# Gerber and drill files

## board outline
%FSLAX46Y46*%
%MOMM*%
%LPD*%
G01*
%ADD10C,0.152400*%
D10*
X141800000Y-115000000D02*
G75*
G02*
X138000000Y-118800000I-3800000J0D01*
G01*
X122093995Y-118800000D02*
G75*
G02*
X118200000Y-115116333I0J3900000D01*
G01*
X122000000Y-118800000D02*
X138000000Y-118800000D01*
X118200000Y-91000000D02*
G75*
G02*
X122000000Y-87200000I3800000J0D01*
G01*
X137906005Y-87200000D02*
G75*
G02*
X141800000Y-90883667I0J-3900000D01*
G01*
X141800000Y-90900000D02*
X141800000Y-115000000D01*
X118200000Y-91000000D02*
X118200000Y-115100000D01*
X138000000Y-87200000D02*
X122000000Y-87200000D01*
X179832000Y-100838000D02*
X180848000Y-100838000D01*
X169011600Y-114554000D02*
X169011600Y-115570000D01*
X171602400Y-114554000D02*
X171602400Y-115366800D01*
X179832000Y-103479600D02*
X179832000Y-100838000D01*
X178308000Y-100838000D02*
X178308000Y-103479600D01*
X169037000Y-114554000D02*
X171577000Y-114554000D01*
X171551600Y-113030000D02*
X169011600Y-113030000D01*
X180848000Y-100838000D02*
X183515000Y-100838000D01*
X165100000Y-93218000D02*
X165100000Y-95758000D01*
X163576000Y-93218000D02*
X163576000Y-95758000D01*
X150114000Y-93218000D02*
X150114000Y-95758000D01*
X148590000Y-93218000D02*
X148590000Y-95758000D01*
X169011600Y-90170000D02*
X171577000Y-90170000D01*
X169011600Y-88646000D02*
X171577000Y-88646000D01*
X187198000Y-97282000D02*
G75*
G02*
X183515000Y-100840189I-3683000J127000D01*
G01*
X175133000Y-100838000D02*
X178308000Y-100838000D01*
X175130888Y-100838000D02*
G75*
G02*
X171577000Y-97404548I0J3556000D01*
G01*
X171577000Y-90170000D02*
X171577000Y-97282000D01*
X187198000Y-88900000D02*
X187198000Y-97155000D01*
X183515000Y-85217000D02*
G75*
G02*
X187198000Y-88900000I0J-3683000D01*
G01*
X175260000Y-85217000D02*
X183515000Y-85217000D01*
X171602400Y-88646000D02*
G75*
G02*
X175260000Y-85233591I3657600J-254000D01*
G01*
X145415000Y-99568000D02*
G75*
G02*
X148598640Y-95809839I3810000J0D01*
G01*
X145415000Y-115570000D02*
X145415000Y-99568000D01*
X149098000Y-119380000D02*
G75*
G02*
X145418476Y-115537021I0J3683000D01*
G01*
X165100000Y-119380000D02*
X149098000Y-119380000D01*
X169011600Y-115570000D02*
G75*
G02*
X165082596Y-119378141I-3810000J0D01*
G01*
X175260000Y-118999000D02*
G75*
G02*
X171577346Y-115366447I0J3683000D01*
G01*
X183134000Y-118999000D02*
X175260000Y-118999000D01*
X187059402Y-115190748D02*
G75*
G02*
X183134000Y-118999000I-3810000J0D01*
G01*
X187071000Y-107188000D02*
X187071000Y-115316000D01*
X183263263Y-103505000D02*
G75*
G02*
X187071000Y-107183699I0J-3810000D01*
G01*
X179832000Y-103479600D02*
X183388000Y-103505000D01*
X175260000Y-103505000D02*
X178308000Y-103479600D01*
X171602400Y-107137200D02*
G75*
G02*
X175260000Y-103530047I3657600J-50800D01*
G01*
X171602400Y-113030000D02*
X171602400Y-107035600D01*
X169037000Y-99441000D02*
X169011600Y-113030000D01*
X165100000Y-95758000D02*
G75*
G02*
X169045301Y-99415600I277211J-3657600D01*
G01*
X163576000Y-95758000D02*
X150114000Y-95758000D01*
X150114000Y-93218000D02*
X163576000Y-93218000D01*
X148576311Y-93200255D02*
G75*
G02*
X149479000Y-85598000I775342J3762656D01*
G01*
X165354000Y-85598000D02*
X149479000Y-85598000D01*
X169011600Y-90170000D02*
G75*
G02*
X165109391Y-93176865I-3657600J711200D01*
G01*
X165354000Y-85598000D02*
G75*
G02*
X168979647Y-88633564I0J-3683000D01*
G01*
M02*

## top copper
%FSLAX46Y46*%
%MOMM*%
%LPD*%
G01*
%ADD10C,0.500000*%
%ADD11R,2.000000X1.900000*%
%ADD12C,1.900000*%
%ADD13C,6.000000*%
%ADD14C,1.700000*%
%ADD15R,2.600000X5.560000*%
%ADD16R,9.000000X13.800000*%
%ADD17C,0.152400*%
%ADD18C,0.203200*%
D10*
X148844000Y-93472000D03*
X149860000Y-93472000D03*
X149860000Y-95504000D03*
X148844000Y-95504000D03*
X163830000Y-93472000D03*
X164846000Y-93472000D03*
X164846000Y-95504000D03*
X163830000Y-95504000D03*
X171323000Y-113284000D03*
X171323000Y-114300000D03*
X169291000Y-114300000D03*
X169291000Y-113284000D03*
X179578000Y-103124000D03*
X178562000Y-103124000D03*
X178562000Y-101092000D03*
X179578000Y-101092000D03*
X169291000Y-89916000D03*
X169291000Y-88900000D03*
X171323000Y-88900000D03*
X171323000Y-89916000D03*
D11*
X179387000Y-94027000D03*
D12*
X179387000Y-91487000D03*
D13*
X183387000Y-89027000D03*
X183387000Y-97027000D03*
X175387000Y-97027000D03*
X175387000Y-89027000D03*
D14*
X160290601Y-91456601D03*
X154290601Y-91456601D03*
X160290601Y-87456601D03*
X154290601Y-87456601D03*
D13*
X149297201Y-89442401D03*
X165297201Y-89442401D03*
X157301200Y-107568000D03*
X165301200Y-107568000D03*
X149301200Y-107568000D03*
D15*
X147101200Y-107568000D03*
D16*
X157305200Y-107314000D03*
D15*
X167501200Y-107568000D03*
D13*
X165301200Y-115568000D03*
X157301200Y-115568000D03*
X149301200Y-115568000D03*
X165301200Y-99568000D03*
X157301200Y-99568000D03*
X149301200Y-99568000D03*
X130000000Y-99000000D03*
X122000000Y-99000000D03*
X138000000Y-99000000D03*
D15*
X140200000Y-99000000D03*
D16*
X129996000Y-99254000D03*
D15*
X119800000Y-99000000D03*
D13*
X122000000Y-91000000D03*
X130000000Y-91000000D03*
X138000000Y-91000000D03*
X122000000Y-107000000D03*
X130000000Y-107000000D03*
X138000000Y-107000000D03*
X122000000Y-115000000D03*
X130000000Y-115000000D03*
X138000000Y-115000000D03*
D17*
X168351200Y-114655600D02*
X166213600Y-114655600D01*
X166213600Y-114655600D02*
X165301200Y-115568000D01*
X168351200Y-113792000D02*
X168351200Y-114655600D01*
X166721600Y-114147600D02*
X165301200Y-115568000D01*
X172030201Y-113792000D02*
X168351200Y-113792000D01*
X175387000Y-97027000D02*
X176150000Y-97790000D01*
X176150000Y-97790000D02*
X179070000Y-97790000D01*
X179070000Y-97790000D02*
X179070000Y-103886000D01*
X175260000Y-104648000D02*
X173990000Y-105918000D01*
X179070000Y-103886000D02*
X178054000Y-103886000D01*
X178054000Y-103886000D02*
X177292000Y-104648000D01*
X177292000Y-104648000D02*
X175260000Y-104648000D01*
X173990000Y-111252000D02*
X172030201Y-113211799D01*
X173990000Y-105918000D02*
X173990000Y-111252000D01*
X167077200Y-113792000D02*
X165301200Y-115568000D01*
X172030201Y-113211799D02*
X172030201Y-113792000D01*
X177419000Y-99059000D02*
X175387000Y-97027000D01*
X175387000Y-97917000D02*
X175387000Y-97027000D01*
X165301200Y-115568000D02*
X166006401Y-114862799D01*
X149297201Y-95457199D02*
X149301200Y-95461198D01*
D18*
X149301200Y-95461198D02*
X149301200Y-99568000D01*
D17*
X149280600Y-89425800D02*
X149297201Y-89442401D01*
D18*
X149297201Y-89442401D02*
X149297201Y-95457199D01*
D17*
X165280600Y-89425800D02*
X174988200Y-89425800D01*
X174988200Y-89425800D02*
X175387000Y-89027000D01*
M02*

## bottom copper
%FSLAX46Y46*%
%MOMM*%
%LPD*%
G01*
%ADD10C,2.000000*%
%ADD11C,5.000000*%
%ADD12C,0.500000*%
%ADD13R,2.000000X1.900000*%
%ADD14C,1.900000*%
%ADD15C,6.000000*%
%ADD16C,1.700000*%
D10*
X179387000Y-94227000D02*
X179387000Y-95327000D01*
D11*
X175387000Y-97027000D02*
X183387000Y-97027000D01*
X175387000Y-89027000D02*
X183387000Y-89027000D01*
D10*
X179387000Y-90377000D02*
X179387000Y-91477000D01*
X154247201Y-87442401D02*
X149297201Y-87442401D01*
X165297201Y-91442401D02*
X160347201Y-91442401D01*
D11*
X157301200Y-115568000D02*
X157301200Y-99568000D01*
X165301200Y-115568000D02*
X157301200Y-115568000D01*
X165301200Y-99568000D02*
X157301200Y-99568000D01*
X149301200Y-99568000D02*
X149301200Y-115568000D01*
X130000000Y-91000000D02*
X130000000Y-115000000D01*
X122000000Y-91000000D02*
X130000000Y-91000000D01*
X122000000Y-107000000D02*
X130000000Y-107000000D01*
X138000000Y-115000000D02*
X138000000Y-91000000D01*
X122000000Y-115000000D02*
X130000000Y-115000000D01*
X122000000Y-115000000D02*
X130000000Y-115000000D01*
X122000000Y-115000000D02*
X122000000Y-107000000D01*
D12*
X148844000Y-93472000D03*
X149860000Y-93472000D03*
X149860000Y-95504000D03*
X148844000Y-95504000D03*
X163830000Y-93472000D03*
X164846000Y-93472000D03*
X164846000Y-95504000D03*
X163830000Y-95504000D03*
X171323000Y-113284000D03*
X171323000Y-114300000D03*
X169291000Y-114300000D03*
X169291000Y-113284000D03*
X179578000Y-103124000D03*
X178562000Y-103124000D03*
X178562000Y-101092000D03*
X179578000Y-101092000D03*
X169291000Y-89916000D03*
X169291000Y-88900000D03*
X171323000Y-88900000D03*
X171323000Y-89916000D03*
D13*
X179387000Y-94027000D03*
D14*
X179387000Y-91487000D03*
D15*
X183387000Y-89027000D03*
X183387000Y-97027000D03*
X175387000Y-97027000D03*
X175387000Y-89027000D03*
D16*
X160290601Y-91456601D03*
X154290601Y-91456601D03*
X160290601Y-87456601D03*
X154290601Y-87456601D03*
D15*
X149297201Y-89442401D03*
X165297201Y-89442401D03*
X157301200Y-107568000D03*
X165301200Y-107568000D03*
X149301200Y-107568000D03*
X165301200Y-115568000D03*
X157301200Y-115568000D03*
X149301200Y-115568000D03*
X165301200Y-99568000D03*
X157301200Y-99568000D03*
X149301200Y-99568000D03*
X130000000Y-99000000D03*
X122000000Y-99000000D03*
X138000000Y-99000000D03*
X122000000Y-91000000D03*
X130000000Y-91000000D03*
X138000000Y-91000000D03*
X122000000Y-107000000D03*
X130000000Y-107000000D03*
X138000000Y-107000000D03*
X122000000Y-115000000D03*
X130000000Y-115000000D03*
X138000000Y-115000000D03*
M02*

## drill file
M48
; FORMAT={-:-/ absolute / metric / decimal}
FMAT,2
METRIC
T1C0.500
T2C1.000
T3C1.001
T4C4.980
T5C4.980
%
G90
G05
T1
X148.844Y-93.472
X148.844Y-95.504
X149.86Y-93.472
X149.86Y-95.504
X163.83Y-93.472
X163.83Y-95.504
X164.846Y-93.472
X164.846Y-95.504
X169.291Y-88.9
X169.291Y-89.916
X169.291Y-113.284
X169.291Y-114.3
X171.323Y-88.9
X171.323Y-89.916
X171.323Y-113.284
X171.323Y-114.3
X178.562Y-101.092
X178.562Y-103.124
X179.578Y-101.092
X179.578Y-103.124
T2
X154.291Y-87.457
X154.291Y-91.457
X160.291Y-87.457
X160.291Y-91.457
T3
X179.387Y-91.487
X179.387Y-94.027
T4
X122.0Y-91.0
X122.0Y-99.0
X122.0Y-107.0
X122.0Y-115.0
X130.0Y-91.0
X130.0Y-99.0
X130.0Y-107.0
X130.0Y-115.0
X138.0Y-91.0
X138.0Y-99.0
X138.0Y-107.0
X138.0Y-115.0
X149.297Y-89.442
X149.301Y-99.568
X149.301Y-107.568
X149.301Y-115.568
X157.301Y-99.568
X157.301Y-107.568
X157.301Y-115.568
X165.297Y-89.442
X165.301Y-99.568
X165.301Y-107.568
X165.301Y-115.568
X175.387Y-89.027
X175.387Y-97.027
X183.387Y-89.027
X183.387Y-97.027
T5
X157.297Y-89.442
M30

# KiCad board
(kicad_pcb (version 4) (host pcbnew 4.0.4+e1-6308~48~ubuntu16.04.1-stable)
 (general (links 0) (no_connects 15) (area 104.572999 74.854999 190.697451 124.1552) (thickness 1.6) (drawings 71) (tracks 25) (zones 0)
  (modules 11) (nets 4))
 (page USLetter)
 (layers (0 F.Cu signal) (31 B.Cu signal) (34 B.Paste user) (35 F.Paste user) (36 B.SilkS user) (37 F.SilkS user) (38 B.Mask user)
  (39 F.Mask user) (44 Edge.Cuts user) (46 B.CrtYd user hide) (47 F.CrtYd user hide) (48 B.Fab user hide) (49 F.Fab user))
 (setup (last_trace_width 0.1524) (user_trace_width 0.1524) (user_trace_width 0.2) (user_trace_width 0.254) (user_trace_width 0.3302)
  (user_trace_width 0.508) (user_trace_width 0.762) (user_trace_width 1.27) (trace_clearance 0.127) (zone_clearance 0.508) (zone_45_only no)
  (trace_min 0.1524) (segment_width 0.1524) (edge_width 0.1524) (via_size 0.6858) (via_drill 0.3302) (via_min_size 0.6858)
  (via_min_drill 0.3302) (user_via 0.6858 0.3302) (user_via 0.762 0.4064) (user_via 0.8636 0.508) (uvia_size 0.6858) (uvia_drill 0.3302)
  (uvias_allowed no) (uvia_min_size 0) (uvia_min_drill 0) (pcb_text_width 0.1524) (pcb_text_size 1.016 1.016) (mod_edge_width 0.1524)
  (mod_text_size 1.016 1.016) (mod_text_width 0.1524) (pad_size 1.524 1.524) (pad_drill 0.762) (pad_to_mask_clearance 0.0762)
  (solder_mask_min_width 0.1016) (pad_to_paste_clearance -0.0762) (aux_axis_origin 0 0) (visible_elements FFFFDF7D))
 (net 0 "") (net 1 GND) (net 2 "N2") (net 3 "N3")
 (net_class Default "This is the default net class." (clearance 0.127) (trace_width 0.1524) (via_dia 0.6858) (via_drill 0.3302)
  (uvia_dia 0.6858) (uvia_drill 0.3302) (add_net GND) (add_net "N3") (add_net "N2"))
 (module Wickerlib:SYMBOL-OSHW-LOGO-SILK (layer F.Cu) (at 179.832 109.982)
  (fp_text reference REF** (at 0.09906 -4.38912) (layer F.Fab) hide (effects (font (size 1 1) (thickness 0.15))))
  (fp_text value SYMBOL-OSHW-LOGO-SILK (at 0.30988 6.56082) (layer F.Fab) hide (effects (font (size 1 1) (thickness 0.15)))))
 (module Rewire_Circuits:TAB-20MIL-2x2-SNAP (layer F.Cu) (at 149.352 94.488)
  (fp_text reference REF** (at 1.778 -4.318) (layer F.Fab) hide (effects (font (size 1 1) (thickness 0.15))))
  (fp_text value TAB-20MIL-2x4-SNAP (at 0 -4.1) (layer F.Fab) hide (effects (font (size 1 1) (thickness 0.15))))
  (pad 1 thru_hole circle (at -0.508 -1.016) (size 0.5 0.5) (drill 0.5) (layers *.Cu))
  (pad 1 thru_hole circle (at 0.508 -1.016) (size 0.5 0.5) (drill 0.5) (layers *.Cu))
  (pad 1 thru_hole circle (at 0.508 1.016) (size 0.5 0.5) (drill 0.5) (layers *.Cu))
  (pad 1 thru_hole circle (at -0.508 1.016) (size 0.5 0.5) (drill 0.5) (layers *.Cu)))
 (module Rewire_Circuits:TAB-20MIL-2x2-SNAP (layer F.Cu) (at 164.338 94.488)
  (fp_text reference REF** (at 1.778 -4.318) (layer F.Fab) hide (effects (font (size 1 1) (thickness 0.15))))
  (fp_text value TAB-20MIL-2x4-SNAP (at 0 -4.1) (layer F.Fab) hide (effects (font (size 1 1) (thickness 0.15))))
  (pad 1 thru_hole circle (at -0.508 -1.016) (size 0.5 0.5) (drill 0.5) (layers *.Cu))
  (pad 1 thru_hole circle (at 0.508 -1.016) (size 0.5 0.5) (drill 0.5) (layers *.Cu))
  (pad 1 thru_hole circle (at 0.508 1.016) (size 0.5 0.5) (drill 0.5) (layers *.Cu))
  (pad 1 thru_hole circle (at -0.508 1.016) (size 0.5 0.5) (drill 0.5) (layers *.Cu)))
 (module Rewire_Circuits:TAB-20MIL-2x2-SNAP (layer F.Cu) (at 170.307 113.792 270)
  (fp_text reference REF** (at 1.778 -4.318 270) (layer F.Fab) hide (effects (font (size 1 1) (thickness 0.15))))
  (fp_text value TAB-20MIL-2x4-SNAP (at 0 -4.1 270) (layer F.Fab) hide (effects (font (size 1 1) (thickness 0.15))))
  (pad 1 thru_hole circle (at -0.508 -1.016 270) (size 0.5 0.5) (drill 0.5) (layers *.Cu))
  (pad 1 thru_hole circle (at 0.508 -1.016 270) (size 0.5 0.5) (drill 0.5) (layers *.Cu))
  (pad 1 thru_hole circle (at 0.508 1.016 270) (size 0.5 0.5) (drill 0.5) (layers *.Cu))
  (pad 1 thru_hole circle (at -0.508 1.016 270) (size 0.5 0.5) (drill 0.5) (layers *.Cu)))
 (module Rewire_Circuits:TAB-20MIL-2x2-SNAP (layer F.Cu) (at 179.07 102.108 180)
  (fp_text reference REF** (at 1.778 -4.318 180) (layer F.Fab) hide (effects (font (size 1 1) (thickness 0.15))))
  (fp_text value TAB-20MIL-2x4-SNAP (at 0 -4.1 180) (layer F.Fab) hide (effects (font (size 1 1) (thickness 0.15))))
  (pad 1 thru_hole circle (at -0.508 -1.016 180) (size 0.5 0.5) (drill 0.5) (layers *.Cu))
  (pad 1 thru_hole circle (at 0.508 -1.016 180) (size 0.5 0.5) (drill 0.5) (layers *.Cu))
  (pad 1 thru_hole circle (at 0.508 1.016 180) (size 0.5 0.5) (drill 0.5) (layers *.Cu))
  (pad 1 thru_hole circle (at -0.508 1.016 180) (size 0.5 0.5) (drill 0.5) (layers *.Cu)))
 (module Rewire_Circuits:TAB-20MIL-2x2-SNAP (layer F.Cu) (at 170.307 89.408 90)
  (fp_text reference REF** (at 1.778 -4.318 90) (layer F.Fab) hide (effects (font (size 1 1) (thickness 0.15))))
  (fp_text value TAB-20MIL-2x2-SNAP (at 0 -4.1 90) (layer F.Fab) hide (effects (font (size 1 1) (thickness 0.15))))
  (pad 1 thru_hole circle (at -0.508 -1.016 90) (size 0.5 0.5) (drill 0.5) (layers *.Cu))
  (pad 1 thru_hole circle (at 0.508 -1.016 90) (size 0.5 0.5) (drill 0.5) (layers *.Cu))
  (pad 1 thru_hole circle (at 0.508 1.016 90) (size 0.5 0.5) (drill 0.5) (layers *.Cu))
  (pad 1 thru_hole circle (at -0.508 1.016 90) (size 0.5 0.5) (drill 0.5) (layers *.Cu)))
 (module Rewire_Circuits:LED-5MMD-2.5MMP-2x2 (layer F.Cu) (at 183.387 89.027 180)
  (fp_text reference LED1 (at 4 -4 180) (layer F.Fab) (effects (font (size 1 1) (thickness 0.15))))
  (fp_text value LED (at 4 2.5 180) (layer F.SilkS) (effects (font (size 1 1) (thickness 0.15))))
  (fp_line (start 4 -5.2) (end 4 -6.3) (layer B.Cu) (width 2)) (fp_line (start 8 -8) (end 0 -8) (layer B.Cu) (width 5))
  (fp_line (start 8 0) (end 0 0) (layer B.Cu) (width 5))
  (fp_line (start 4 -1.35) (end 4 -2.45) (layer B.Cu) (width 2))
  (pad - thru_hole rect (at 4 -5 180) (size 2 1.9) (drill 1.00076) (layers *.Cu *.Mask) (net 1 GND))
  (pad + thru_hole circle (at 4 -2.46 90) (size 1.9 1.9) (drill 1.00076) (layers *.Cu *.Mask) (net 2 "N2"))
  (pad + thru_hole circle (at 0 0 180) (size 6 6) (drill 4.98) (layers *.Cu *.Mask) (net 2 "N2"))
  (pad - thru_hole circle (at 0 -8 180) (size 6 6) (drill 4.98) (layers *.Cu *.Mask) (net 1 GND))
  (pad - thru_hole circle (at 8 -8 180) (size 6 6) (drill 4.98) (layers *.Cu *.Mask) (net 1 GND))
  (pad + thru_hole circle (at 8 0 180) (size 6 6) (drill 4.98) (layers *.Cu *.Mask) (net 2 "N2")))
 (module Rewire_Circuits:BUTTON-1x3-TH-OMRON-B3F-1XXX (layer F.Cu) (at 149.297201 89.442401)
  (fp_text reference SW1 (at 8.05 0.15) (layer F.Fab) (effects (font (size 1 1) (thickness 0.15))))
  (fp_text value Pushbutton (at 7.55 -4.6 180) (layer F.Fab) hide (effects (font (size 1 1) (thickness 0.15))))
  (fp_line (start 4.95 -2) (end 0 -2) (layer B.Cu) (width 2)) (fp_line (start 16 2) (end 11.05 2) (layer B.Cu) (width 2))
  (pad 2 thru_hole circle (at 10.9934 2.0142) (size 1.7 1.7) (drill 1) (layers *.Cu *.Mask) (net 2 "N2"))
  (pad 2 thru_hole circle (at 4.9934 2.0142) (size 1.7 1.7) (drill 1) (layers *.Cu *.Mask) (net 2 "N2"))
  (pad 1 thru_hole circle (at 10.9934 -1.9858) (size 1.7 1.7) (drill 1) (layers *.Cu *.Mask) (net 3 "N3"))
  (pad 1 thru_hole circle (at 4.9934 -1.9858) (size 1.7 1.7) (drill 1) (layers *.Cu *.Mask) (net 3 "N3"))
  (pad "" np_thru_hole circle (at 8 0) (size 4.88 4.88) (drill 4.98) (layers *.Cu *.Mask F.SilkS))
  (pad 1 thru_hole circle (at 0 0) (size 6 6) (drill 4.98) (layers *.Cu *.Mask F.SilkS) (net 3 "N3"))
  (pad 2 thru_hole circle (at 16 0) (size 6 6) (drill 4.98) (layers *.Cu *.Mask F.SilkS) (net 2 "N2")))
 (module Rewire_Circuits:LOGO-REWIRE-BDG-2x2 (layer F.Cu) (at 179.324 111.252)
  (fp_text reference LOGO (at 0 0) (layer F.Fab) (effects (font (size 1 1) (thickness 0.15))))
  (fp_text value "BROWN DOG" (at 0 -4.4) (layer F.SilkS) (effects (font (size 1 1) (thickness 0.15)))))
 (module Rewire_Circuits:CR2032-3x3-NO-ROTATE (layer F.Cu) (at 165.3012 99.568 180)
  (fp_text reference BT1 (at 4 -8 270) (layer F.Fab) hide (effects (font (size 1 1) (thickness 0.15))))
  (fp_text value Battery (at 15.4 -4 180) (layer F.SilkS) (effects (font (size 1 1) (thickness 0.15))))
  (fp_line (start 8 -16) (end 8 0) (layer B.Cu) (width 5)) (fp_line (start 0 -16) (end 8 -16) (layer B.Cu) (width 5))
  (fp_line (start 0 0) (end 8 0) (layer B.Cu) (width 5)) (fp_line (start 16 0) (end 16 -16) (layer B.Cu) (width 5))
  (pad GND thru_hole circle (at 8 -8 180) (size 6 6) (drill 4.98) (layers *.Cu *.Mask) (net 1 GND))
  (pad + thru_hole circle (at 0 -8 180) (size 6 6) (drill 4.98) (layers *.Cu) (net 3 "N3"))
  (pad + thru_hole circle (at 16 -8 180) (size 6 6) (drill 4.98) (layers *.Cu B.Mask) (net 3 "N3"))
  (pad + smd rect (at 18.2 -8 180) (size 2.6 5.56) (layers F.Cu F.Paste F.Mask) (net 3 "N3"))
  (pad GND smd rect (at 7.996 -7.746 180) (size 9 13.8) (layers F.Cu F.Paste F.Mask) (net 1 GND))
  (pad + smd rect (at -2.2 -8 180) (size 2.6 5.56) (layers F.Cu F.Paste F.Mask) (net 3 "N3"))
  (pad GND thru_hole circle (at 0 -16 180) (size 6 6) (drill 4.98) (layers *.Cu *.Mask) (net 1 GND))
  (pad GND thru_hole circle (at 8 -16 180) (size 6 6) (drill 4.98) (layers *.Cu *.Mask) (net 1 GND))
  (pad + thru_hole circle (at 16 -16 180) (size 6 6) (drill 4.98) (layers *.Cu B.Mask) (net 3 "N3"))
  (pad GND thru_hole circle (at 0 0 180) (size 6 6) (drill 4.98) (layers *.Cu *.Mask) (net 1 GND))
  (pad GND thru_hole circle (at 8 0 180) (size 6 6) (drill 4.98) (layers *.Cu *.Mask) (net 1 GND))
  (pad + thru_hole circle (at 16 0 180) (size 6 6) (drill 4.98) (layers *.Cu B.Mask) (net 3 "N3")))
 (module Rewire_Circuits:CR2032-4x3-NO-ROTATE (layer F.Cu) (at 122 107)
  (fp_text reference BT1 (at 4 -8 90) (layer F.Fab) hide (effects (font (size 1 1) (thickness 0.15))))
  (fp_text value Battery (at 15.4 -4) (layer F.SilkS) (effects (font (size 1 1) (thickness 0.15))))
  (fp_line (start 8 -16) (end 8 8) (layer B.Cu) (width 5)) (fp_line (start 0 -16) (end 8 -16) (layer B.Cu) (width 5))
  (fp_line (start 0 0) (end 8 0) (layer B.Cu) (width 5)) (fp_line (start 16 8) (end 16 -16) (layer B.Cu) (width 5))
  (fp_line (start 0 8) (end 8 8) (layer B.Cu) (width 5)) (fp_line (start 0 8) (end 8 8) (layer B.Cu) (width 5))
  (fp_line (start 0 8) (end 0 0) (layer B.Cu) (width 5))
  (pad GND thru_hole circle (at 8 -8) (size 6 6) (drill 4.98) (layers *.Cu *.Mask))
  (pad + thru_hole circle (at 0 -8) (size 6 6) (drill 4.98) (layers *.Cu))
  (pad + thru_hole circle (at 16 -8) (size 6 6) (drill 4.98) (layers *.Cu B.Mask))
  (pad + smd rect (at 18.2 -8) (size 2.6 5.56) (layers F.Cu F.Paste F.Mask))
  (pad GND smd rect (at 7.996 -7.746) (size 9 13.8) (layers F.Cu F.Paste F.Mask))
  (pad + smd rect (at -2.2 -8) (size 2.6 5.56) (layers F.Cu F.Paste F.Mask))
  (pad GND thru_hole circle (at 0 -16) (size 6 6) (drill 4.98) (layers *.Cu *.Mask))
  (pad GND thru_hole circle (at 8 -16) (size 6 6) (drill 4.98) (layers *.Cu *.Mask))
  (pad + thru_hole circle (at 16 -16) (size 6 6) (drill 4.98) (layers *.Cu B.Mask))
  (pad GND thru_hole circle (at 0 0) (size 6 6) (drill 4.98) (layers *.Cu *.Mask))
  (pad GND thru_hole circle (at 8 0) (size 6 6) (drill 4.98) (layers *.Cu *.Mask))
  (pad + thru_hole circle (at 16 0) (size 6 6) (drill 4.98) (layers *.Cu B.Mask))
  (pad GND thru_hole circle (at 0 8) (size 6 6) (drill 4.98) (layers *.Cu *.Mask))
  (pad GND thru_hole circle (at 8 8) (size 6 6) (drill 4.98) (layers *.Cu *.Mask))
  (pad + thru_hole circle (at 16 8) (size 6 6) (drill 4.98) (layers *.Cu B.Mask)))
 (gr_arc (start 138 115) (end 141.8 115) (angle 90) (layer Edge.Cuts) (width 0.1524))
 (gr_arc (start 122.093995 114.9) (end 122.093995 118.8) (angle 86.82016988) (layer Edge.Cuts) (width 0.1524))
 (gr_line (start 122 118.8) (end 138 118.8) (layer Edge.Cuts) (width 0.1524))
 (gr_arc (start 122 91) (end 118.2 91) (angle 90) (layer Edge.Cuts) (width 0.1524))
 (gr_arc (start 137.906005 91.1) (end 137.906005 87.2) (angle 86.82016988) (layer Edge.Cuts) (width 0.1524))
 (gr_line (start 141.8 90.9) (end 141.8 115) (layer Edge.Cuts) (width 0.1524))
 (gr_line (start 118.2 91) (end 118.2 115.1) (layer Edge.Cuts) (width 0.1524))
 (gr_line (start 138 87.2) (end 122 87.2) (layer Edge.Cuts) (width 0.1524))
 (gr_line (start 179.832 100.838) (end 180.848 100.838) (layer Edge.Cuts) (width 0.1524))
 (gr_line (start 169.0116 114.554) (end 169.0116 115.57) (layer Edge.Cuts) (width 0.1524))
 (gr_line (start 171.6024 114.554) (end 171.6024 115.3668) (layer Edge.Cuts) (width 0.1524))
 (gr_line (start 179.832 103.4796) (end 179.832 100.838) (layer Edge.Cuts) (width 0.1524))
 (gr_line (start 178.308 100.838) (end 178.308 103.4796) (layer Edge.Cuts) (width 0.1524))
 (gr_line (start 169.037 114.554) (end 171.577 114.554) (layer Edge.Cuts) (width 0.1524))
 (gr_line (start 171.5516 113.03) (end 169.0116 113.03) (layer Edge.Cuts) (width 0.1524))
 (gr_line (start 180.848 100.838) (end 183.515 100.838) (layer Edge.Cuts) (width 0.1524))
 (gr_line (start 165.1 93.218) (end 165.1 95.758) (layer Edge.Cuts) (width 0.1524))
 (gr_line (start 163.576 93.218) (end 163.576 95.758) (layer Edge.Cuts) (width 0.1524))
 (gr_line (start 150.114 93.218) (end 150.114 95.758) (layer Edge.Cuts) (width 0.1524))
 (gr_line (start 148.59 93.218) (end 148.59 95.758) (layer Edge.Cuts) (width 0.1524))
 (gr_line (start 169.0116 90.17) (end 171.577 90.17) (layer Edge.Cuts) (width 0.1524))
 (gr_line (start 169.0116 88.646) (end 171.577 88.646) (layer Edge.Cuts) (width 0.1524))
 (gr_arc (start 183.515 97.155) (end 187.198 97.282) (angle 88.02506599) (layer Edge.Cuts) (width 0.1524))
 (gr_line (start 175.133 100.838) (end 178.308 100.838) (layer Edge.Cuts) (width 0.1524))
 (gr_arc (start 175.130888 97.282) (end 175.130888 100.838) (angle 88.02506599) (layer Edge.Cuts) (width 0.1524))
 (gr_line (start 171.577 90.17) (end 171.577 97.282) (layer Edge.Cuts) (width 0.1524))
 (gr_line (start 187.198 88.9) (end 187.198 97.155) (layer Edge.Cuts) (width 0.1524))
 (gr_arc (start 183.515 88.9) (end 183.515 85.217) (angle 90) (layer Edge.Cuts) (width 0.1524))
 (gr_line (start 175.26 85.217) (end 183.515 85.217) (layer Edge.Cuts) (width 0.1524))
 (gr_arc (start 175.26 88.9) (end 171.6024 88.646) (angle 86.02750406) (layer Edge.Cuts) (width 0.1524))
 (gr_arc (start 149.225 99.568) (end 145.415 99.568) (angle 80.53767779) (layer Edge.Cuts) (width 0.1524))
 (gr_line (start 145.415 115.57) (end 145.415 99.568) (layer Edge.Cuts) (width 0.1524))
 (gr_arc (start 149.098 115.697) (end 149.098 119.38) (angle 92.48955292) (layer Edge.Cuts) (width 0.1524))
 (gr_line (start 165.1 119.38) (end 149.098 119.38) (layer Edge.Cuts) (width 0.1524))
 (gr_arc (start 165.2016 115.57) (end 169.0116 115.57) (angle 91.7899045) (layer Edge.Cuts) (width 0.1524))
 (gr_arc (start 175.26 115.316) (end 175.26 118.999) (angle 89.2151803) (layer Edge.Cuts) (width 0.1524))
 (gr_line (start 183.134 118.999) (end 175.26 118.999) (layer Edge.Cuts) (width 0.1524))
 (gr_arc (start 183.249402 115.190748) (end 187.059402 115.190748) (angle 91.73570459) (layer Edge.Cuts) (width 0.1524))
 (gr_line (start 187.071 107.188) (end 187.071 115.316) (layer Edge.Cuts) (width 0.1524))
 (gr_arc (start 183.263263 107.315) (end 183.263263 103.505) (angle 88.02506599) (layer Edge.Cuts) (width 0.1524))
 (gr_line (start 179.832 103.4796) (end 183.388 103.505) (layer Edge.Cuts) (width 0.1524))
 (gr_line (start 175.26 103.505) (end 178.308 103.4796) (layer Edge.Cuts) (width 0.1524))
 (gr_arc (start 175.26 107.188) (end 171.6024 107.1372) (angle 89.20427645) (layer Edge.Cuts) (width 0.1524))
 (gr_line (start 171.6024 113.03) (end 171.6024 107.0356) (layer Edge.Cuts) (width 0.1524))
 (gr_line (start 169.037 99.441) (end 169.0116 113.03) (layer Edge.Cuts) (width 0.1524))
 (gr_arc (start 165.377211 99.4156) (end 165.1 95.758) (angle 94.33418445) (layer Edge.Cuts) (width 0.1524))
 (gr_line (start 163.576 95.758) (end 150.114 95.758) (layer Edge.Cuts) (width 0.1524))
 (gr_line (start 150.114 93.218) (end 163.576 93.218) (layer Edge.Cuts) (width 0.1524))
 (gr_arc (start 149.351653 89.437599) (end 148.576311 93.200255) (angle 170.256088) (layer Edge.Cuts) (width 0.1524))
 (gr_line (start 165.354 85.598) (end 149.479 85.598) (layer Edge.Cuts) (width 0.1524))
 (gr_arc (start 165.354 89.4588) (end 169.0116 90.17) (angle 82.76048574) (layer Edge.Cuts) (width 0.1524))
 (gr_arc (start 165.354 89.281) (end 165.354 85.598) (angle 79.87534038) (layer Edge.Cuts) (width 0.1524))
 (segment (start 168.3512 114.6556) (end 166.2136 114.6556) (width 0.1524) (layer F.Cu) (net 1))
 (segment (start 166.2136 114.6556) (end 165.3012 115.568) (width 0.1524) (layer F.Cu) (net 1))
 (segment (start 168.3512 113.792) (end 168.3512 114.6556) (width 0.1524) (layer F.Cu) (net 1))
 (segment (start 166.7216 114.1476) (end 165.3012 115.568) (width 0.1524) (layer F.Cu) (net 1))
 (segment (start 172.030201 113.792) (end 168.3512 113.792) (width 0.1524) (layer F.Cu) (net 1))
 (segment (start 175.387 97.027) (end 176.15 97.79) (width 0.1524) (layer F.Cu) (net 1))
 (segment (start 176.15 97.79) (end 179.07 97.79) (width 0.1524) (layer F.Cu) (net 1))
 (segment (start 179.07 97.79) (end 179.07 103.886) (width 0.1524) (layer F.Cu) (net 1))
 (segment (start 175.26 104.648) (end 173.99 105.918) (width 0.1524) (layer F.Cu) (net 1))
 (segment (start 179.07 103.886) (end 178.054 103.886) (width 0.1524) (layer F.Cu) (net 1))
 (segment (start 178.054 103.886) (end 177.292 104.648) (width 0.1524) (layer F.Cu) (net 1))
 (segment (start 177.292 104.648) (end 175.26 104.648) (width 0.1524) (layer F.Cu) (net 1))
 (segment (start 173.99 111.252) (end 172.030201 113.211799) (width 0.1524) (layer F.Cu) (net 1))
 (segment (start 173.99 105.918) (end 173.99 111.252) (width 0.1524) (layer F.Cu) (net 1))
 (segment (start 167.0772 113.792) (end 165.3012 115.568) (width 0.1524) (layer F.Cu) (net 1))
 (segment (start 172.030201 113.211799) (end 172.030201 113.792) (width 0.1524) (layer F.Cu) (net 1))
 (segment (start 177.419 99.059) (end 175.387 97.027) (width 0.1524) (layer F.Cu) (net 1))
 (segment (start 175.387 97.917) (end 175.387 97.027) (width 0.1524) (layer F.Cu) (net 1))
 (segment (start 165.3012 115.568) (end 166.006401 114.862799) (width 0.1524) (layer F.Cu) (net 1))
 (segment (start 149.297201 95.457199) (end 149.3012 95.461198) (width 0.1524) (layer F.Cu) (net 3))
 (segment (start 149.3012 95.461198) (end 149.3012 99.568) (width 0.2032) (layer F.Cu) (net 3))
 (segment (start 149.2806 89.4258) (end 149.297201 89.442401) (width 0.1524) (layer F.Cu) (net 3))
 (segment (start 149.297201 89.442401) (end 149.297201 95.457199) (width 0.2032) (layer F.Cu) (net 3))
 (segment (start 165.2806 89.4258) (end 174.9882 89.4258) (width 0.1524) (layer F.Cu) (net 2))
 (segment (start 174.9882 89.4258) (end 175.387 89.027) (width 0.1524) (layer F.Cu) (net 2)))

